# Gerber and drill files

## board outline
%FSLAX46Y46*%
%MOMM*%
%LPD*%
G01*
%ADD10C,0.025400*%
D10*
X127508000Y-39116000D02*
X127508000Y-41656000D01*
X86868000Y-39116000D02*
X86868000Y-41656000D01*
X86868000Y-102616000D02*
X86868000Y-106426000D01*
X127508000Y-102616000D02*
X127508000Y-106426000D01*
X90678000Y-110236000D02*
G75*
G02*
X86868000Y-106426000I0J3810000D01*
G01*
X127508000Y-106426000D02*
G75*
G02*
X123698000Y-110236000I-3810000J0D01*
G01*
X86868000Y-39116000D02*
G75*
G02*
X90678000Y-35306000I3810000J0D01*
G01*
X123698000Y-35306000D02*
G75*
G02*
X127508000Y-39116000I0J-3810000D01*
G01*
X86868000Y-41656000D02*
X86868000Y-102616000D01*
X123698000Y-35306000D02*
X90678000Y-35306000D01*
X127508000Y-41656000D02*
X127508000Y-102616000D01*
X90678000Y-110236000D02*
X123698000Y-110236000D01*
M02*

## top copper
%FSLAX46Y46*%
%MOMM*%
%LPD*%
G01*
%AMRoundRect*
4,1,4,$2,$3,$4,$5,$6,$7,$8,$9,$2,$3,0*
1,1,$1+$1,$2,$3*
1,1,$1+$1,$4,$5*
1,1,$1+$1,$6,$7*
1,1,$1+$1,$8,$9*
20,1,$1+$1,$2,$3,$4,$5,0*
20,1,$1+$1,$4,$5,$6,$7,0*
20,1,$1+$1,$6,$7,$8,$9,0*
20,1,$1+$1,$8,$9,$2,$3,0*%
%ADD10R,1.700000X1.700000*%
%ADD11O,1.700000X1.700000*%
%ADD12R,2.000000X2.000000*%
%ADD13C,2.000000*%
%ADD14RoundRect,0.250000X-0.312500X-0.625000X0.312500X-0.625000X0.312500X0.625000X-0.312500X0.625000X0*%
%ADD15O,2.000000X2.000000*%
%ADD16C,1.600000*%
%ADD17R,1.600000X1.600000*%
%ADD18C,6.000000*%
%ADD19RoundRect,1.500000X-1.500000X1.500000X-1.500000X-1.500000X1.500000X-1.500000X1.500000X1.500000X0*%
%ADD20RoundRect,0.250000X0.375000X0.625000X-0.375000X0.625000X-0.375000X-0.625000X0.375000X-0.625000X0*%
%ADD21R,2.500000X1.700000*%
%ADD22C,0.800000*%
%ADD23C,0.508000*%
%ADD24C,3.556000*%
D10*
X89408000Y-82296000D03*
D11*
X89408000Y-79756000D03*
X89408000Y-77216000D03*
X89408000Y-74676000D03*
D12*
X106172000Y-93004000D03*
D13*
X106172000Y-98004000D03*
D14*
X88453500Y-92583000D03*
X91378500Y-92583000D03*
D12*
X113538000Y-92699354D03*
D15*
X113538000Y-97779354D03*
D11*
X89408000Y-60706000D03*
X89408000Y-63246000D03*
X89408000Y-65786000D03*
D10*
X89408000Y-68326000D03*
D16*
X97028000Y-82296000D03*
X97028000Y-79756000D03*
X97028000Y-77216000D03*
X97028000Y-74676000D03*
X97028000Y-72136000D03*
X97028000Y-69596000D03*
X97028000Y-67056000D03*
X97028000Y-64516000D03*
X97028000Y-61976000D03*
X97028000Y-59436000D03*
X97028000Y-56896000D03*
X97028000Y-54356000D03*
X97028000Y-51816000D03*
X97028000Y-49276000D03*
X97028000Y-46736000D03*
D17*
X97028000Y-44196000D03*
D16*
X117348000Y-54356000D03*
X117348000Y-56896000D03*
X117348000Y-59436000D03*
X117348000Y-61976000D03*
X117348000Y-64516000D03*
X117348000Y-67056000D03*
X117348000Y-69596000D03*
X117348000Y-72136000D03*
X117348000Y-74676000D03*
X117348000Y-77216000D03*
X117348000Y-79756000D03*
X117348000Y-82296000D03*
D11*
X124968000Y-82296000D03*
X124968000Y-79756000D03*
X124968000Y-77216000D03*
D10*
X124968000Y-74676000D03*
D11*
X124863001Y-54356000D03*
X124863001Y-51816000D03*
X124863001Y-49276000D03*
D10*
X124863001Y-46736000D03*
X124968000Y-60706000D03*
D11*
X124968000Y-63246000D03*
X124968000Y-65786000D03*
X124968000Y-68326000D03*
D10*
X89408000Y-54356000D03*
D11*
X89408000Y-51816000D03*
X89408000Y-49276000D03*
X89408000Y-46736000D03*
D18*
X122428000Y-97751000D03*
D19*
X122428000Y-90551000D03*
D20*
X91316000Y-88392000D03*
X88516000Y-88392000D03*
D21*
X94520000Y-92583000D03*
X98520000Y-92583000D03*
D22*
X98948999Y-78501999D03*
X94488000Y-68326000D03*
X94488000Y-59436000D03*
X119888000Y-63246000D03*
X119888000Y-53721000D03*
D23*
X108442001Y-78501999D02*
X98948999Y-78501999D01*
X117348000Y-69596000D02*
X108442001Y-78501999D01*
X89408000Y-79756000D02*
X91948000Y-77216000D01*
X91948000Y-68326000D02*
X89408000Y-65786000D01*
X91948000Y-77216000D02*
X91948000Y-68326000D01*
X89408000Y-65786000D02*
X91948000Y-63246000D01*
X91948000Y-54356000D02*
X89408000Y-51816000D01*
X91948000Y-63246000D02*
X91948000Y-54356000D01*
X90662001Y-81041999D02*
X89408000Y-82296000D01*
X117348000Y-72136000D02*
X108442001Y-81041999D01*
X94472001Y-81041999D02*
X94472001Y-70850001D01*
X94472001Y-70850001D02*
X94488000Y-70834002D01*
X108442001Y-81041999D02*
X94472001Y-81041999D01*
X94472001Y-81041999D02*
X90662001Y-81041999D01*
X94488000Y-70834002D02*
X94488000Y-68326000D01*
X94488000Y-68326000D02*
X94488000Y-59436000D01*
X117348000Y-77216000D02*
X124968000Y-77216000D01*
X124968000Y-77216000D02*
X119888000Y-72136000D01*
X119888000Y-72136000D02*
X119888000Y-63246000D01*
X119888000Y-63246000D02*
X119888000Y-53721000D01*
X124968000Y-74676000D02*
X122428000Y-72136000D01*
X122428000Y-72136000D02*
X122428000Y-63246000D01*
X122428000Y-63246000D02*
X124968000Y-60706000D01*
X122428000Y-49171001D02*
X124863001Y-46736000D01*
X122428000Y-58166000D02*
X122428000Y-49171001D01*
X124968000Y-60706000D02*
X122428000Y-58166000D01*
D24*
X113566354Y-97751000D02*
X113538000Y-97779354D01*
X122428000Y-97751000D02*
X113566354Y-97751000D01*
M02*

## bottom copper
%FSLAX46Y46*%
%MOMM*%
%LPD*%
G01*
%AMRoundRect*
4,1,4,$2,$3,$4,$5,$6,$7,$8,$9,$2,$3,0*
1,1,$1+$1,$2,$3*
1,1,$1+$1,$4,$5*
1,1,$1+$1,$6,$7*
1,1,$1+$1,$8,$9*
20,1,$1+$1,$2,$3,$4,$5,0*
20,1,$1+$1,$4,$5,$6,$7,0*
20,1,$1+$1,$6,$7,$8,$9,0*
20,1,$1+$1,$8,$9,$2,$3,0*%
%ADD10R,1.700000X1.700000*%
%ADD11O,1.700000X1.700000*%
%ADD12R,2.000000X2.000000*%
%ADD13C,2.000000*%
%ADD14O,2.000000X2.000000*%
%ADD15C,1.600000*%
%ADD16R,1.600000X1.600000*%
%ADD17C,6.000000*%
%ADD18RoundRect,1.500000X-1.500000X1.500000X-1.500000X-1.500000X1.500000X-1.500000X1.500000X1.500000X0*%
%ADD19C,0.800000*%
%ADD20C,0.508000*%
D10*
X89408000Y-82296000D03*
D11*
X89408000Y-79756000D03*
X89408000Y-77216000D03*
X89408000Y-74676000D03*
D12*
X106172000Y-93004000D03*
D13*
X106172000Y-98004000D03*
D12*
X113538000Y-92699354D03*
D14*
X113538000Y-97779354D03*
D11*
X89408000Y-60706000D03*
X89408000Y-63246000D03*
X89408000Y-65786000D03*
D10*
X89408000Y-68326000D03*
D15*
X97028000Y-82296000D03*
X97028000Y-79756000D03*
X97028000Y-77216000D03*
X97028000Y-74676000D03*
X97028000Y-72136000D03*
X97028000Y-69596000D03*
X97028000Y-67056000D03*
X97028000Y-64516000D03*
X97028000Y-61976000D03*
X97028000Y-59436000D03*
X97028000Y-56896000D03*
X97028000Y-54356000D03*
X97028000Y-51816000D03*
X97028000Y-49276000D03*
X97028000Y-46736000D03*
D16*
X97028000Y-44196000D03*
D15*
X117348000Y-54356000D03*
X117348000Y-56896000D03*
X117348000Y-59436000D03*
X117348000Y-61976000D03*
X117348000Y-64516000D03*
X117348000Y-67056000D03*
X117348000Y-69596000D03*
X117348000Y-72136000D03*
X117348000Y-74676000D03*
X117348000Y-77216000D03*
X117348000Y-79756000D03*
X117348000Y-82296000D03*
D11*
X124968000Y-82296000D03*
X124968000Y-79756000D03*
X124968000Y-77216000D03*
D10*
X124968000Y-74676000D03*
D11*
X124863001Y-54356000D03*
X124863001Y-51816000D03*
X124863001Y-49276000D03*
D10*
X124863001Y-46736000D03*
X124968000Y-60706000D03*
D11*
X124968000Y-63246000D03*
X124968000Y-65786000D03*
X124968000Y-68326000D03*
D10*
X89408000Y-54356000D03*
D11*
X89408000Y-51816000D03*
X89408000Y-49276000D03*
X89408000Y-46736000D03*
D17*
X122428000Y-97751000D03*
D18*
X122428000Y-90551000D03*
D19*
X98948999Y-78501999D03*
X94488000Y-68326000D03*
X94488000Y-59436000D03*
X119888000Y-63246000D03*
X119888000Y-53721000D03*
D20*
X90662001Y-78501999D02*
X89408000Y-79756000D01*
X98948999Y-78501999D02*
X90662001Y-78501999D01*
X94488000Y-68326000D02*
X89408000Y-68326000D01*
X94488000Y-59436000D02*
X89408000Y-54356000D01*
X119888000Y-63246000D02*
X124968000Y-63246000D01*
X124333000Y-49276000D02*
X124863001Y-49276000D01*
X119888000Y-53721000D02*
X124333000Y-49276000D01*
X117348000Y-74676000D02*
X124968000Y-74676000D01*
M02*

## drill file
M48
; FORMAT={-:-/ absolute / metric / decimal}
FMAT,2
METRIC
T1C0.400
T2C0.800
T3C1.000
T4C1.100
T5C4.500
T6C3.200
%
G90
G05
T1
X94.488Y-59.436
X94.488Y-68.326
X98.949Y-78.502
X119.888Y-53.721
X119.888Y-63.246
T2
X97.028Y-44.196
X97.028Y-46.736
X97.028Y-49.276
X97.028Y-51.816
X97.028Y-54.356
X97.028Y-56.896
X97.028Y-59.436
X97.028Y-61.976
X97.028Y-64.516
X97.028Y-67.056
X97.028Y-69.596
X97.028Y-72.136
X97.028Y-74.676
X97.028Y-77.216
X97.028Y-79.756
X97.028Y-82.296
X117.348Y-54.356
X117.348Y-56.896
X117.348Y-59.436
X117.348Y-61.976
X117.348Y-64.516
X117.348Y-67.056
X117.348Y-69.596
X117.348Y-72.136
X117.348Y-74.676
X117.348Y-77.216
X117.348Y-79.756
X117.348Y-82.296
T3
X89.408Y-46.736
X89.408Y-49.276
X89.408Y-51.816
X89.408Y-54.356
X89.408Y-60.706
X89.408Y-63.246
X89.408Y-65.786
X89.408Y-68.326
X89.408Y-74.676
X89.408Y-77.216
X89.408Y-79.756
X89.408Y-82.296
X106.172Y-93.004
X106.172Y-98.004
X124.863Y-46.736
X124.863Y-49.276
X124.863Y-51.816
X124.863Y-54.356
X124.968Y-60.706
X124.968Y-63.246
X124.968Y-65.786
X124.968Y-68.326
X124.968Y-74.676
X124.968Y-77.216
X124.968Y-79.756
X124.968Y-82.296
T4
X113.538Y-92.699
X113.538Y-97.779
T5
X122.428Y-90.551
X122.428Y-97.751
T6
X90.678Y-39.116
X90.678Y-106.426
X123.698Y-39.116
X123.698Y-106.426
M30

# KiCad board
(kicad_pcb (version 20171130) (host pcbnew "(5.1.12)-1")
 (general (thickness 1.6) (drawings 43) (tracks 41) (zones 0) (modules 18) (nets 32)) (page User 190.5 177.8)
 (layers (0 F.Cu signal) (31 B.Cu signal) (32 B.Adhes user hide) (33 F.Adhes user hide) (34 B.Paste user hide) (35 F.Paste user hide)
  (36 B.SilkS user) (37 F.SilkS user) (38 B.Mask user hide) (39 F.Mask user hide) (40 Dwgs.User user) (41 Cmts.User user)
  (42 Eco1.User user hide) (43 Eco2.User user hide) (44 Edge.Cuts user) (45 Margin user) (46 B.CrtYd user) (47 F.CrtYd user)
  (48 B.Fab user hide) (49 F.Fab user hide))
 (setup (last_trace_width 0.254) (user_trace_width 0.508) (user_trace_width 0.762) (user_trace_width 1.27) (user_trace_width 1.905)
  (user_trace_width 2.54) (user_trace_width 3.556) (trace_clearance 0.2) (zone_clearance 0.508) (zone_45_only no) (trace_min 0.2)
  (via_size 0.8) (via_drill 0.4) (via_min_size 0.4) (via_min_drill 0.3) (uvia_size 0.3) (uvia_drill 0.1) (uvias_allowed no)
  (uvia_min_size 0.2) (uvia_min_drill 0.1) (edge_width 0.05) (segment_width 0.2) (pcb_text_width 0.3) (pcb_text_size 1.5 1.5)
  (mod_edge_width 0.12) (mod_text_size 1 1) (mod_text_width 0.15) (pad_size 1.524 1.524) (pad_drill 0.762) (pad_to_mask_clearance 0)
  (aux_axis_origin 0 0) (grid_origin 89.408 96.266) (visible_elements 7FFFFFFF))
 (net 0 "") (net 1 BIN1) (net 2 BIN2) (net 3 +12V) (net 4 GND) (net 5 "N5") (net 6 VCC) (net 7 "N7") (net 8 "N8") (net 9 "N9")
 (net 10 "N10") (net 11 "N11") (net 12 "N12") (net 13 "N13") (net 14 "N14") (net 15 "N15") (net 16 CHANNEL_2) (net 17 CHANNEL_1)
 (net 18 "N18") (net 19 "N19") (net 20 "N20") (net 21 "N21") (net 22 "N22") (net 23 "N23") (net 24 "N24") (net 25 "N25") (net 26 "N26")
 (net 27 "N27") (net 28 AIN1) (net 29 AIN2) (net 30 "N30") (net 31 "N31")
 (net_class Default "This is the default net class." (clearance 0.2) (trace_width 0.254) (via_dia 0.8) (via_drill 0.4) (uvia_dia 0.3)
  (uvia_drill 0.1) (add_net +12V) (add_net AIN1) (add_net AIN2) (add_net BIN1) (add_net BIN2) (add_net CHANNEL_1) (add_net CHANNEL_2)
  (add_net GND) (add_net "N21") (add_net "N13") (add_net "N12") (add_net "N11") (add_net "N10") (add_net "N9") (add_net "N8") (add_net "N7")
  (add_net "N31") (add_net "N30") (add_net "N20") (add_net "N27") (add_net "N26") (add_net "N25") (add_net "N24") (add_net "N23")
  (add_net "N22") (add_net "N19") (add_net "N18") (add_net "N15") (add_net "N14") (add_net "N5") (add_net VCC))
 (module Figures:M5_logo (layer F.Cu) (at 99.568 105.405088)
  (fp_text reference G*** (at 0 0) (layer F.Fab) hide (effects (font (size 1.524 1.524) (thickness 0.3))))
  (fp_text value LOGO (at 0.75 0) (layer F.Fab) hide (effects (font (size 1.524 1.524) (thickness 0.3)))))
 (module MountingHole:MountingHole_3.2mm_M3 (layer F.Cu) (at 123.698 39.116)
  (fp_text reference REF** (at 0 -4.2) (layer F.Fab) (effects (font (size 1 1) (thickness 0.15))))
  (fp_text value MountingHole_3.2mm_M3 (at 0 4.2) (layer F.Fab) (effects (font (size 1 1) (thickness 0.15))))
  (pad 1 np_thru_hole circle (at 0 0) (size 3.2 3.2) (drill 3.2) (layers *.Cu *.Mask)))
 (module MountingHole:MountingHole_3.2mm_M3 (layer F.Cu) (at 90.678 39.116)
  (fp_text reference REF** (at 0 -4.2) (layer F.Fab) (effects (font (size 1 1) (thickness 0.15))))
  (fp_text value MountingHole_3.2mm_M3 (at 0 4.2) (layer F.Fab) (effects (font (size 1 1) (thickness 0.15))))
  (pad 1 np_thru_hole circle (at 0 0) (size 3.2 3.2) (drill 3.2) (layers *.Cu *.Mask)))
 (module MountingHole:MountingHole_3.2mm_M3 (layer F.Cu) (at 123.698 106.426)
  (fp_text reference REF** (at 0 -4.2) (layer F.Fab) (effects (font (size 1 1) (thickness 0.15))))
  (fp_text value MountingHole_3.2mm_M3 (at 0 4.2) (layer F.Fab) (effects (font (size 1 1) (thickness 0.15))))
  (pad 1 np_thru_hole circle (at 0 0) (size 3.2 3.2) (drill 3.2) (layers *.Cu *.Mask)))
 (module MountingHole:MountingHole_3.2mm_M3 (layer F.Cu) (at 90.678 106.426)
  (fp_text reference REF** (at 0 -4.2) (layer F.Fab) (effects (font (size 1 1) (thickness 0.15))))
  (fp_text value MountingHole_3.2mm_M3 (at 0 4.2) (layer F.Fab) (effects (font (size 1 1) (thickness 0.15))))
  (pad 1 np_thru_hole circle (at 0 0) (size 3.2 3.2) (drill 3.2) (layers *.Cu *.Mask)))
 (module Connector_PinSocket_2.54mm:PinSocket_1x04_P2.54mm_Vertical (layer F.Cu) (at 89.408 82.296 180)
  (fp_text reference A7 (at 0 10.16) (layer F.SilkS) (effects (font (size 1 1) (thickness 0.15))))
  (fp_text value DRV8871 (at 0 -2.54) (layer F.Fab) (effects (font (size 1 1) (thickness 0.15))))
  (pad 1 thru_hole rect (at 0 0 180) (size 1.7 1.7) (drill 1) (layers *.Cu *.Mask) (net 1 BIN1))
  (pad 2 thru_hole oval (at 0 2.54 180) (size 1.7 1.7) (drill 1) (layers *.Cu *.Mask) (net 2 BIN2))
  (pad 3 thru_hole oval (at 0 5.08 180) (size 1.7 1.7) (drill 1) (layers *.Cu *.Mask) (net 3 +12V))
  (pad 4 thru_hole oval (at 0 7.62 180) (size 1.7 1.7) (drill 1) (layers *.Cu *.Mask) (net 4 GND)))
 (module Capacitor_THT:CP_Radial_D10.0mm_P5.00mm (layer F.Cu) (at 106.172 93.004 270)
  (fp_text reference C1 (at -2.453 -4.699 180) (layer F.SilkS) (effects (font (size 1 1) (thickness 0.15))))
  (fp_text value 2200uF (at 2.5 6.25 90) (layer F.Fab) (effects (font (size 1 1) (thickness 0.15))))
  (pad 1 thru_hole rect (at 0 0 270) (size 2 2) (drill 1) (layers *.Cu *.Mask) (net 3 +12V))
  (pad 2 thru_hole circle (at 5 0 270) (size 2 2) (drill 1) (layers *.Cu *.Mask) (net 4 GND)))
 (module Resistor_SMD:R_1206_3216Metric (layer F.Cu) (at 89.916 92.583)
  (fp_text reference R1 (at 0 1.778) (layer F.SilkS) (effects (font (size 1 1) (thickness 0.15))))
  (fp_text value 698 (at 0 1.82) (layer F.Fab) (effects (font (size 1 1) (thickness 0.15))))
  (pad 1 smd roundrect (at -1.4625 0) (size 1.125 1.75) (layers F.Cu F.Paste F.Mask) (roundrect_rratio 0.222222) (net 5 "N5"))
  (pad 2 smd roundrect (at 1.4625 0) (size 1.125 1.75) (layers F.Cu F.Paste F.Mask) (roundrect_rratio 0.222222) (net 3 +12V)))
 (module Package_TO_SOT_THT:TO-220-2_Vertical (layer F.Cu) (at 113.538 92.699354 270)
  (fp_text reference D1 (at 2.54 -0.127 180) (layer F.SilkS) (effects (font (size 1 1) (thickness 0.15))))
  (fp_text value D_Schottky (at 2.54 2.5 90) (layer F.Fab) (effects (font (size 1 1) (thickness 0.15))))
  (pad 1 thru_hole rect (at 0 0 270) (size 2 2) (drill 1.1) (layers *.Cu *.Mask) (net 3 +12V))
  (pad 2 thru_hole oval (at 5.08 0 270) (size 2 2) (drill 1.1) (layers *.Cu *.Mask) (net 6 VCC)))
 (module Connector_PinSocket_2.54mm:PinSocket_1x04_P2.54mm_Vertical (layer F.Cu) (at 89.408 68.326 180)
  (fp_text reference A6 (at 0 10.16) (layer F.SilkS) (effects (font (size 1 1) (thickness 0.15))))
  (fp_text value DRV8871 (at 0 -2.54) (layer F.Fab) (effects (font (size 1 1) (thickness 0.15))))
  (pad 4 thru_hole oval (at 0 7.62 180) (size 1.7 1.7) (drill 1) (layers *.Cu *.Mask) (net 4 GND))
  (pad 3 thru_hole oval (at 0 5.08 180) (size 1.7 1.7) (drill 1) (layers *.Cu *.Mask) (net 3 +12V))
  (pad 2 thru_hole oval (at 0 2.54 180) (size 1.7 1.7) (drill 1) (layers *.Cu *.Mask) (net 2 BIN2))
  (pad 1 thru_hole rect (at 0 0 180) (size 1.7 1.7) (drill 1) (layers *.Cu *.Mask) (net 1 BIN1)))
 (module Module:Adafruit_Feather (layer F.Cu) (at 97.028 44.196)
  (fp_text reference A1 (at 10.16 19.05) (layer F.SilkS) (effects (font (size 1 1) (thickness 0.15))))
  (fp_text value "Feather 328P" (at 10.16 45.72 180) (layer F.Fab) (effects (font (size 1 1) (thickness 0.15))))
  (pad 16 thru_hole circle (at 0 38.1 180) (size 1.6 1.6) (drill 0.8) (layers *.Cu *.Mask) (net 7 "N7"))
  (pad 15 thru_hole circle (at 0 35.56 180) (size 1.6 1.6) (drill 0.8) (layers *.Cu *.Mask) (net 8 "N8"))
  (pad 14 thru_hole circle (at 0 33.02 180) (size 1.6 1.6) (drill 0.8) (layers *.Cu *.Mask) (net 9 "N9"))
  (pad 13 thru_hole circle (at 0 30.48 180) (size 1.6 1.6) (drill 0.8) (layers *.Cu *.Mask) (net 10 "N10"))
  (pad 12 thru_hole circle (at 0 27.94 180) (size 1.6 1.6) (drill 0.8) (layers *.Cu *.Mask) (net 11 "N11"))
  (pad 11 thru_hole circle (at 0 25.4 180) (size 1.6 1.6) (drill 0.8) (layers *.Cu *.Mask) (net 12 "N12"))
  (pad 10 thru_hole circle (at 0 22.86 180) (size 1.6 1.6) (drill 0.8) (layers *.Cu *.Mask) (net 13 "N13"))
  (pad 9 thru_hole circle (at 0 20.32 180) (size 1.6 1.6) (drill 0.8) (layers *.Cu *.Mask) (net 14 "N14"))
  (pad 8 thru_hole circle (at 0 17.78 180) (size 1.6 1.6) (drill 0.8) (layers *.Cu *.Mask) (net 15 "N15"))
  (pad 7 thru_hole circle (at 0 15.24 180) (size 1.6 1.6) (drill 0.8) (layers *.Cu *.Mask) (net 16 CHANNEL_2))
  (pad 6 thru_hole circle (at 0 12.7 180) (size 1.6 1.6) (drill 0.8) (layers *.Cu *.Mask) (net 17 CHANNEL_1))
  (pad 5 thru_hole circle (at 0 10.16 180) (size 1.6 1.6) (drill 0.8) (layers *.Cu *.Mask) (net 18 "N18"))
  (pad 4 thru_hole circle (at 0 7.62 180) (size 1.6 1.6) (drill 0.8) (layers *.Cu *.Mask) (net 4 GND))
  (pad 3 thru_hole circle (at 0 5.08 180) (size 1.6 1.6) (drill 0.8) (layers *.Cu *.Mask) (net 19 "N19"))
  (pad 2 thru_hole circle (at 0 2.54 180) (size 1.6 1.6) (drill 0.8) (layers *.Cu *.Mask) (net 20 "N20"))
  (pad 1 thru_hole rect (at 0 0 180) (size 1.6 1.6) (drill 0.8) (layers *.Cu *.Mask) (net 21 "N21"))
  (pad 28 thru_hole circle (at 20.32 10.16 180) (size 1.6 1.6) (drill 0.8) (layers *.Cu *.Mask) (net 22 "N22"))
  (pad 27 thru_hole circle (at 20.32 12.7 180) (size 1.6 1.6) (drill 0.8) (layers *.Cu *.Mask) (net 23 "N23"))
  (pad 26 thru_hole circle (at 20.32 15.24 180) (size 1.6 1.6) (drill 0.8) (layers *.Cu *.Mask) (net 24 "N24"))
  (pad 25 thru_hole circle (at 20.32 17.78 180) (size 1.6 1.6) (drill 0.8) (layers *.Cu *.Mask) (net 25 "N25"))
  (pad 24 thru_hole circle (at 20.32 20.32 180) (size 1.6 1.6) (drill 0.8) (layers *.Cu *.Mask) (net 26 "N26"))
  (pad 23 thru_hole circle (at 20.32 22.86 180) (size 1.6 1.6) (drill 0.8) (layers *.Cu *.Mask) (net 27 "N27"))
  (pad 22 thru_hole circle (at 20.32 25.4 180) (size 1.6 1.6) (drill 0.8) (layers *.Cu *.Mask) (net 2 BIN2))
  (pad 21 thru_hole circle (at 20.32 27.94 180) (size 1.6 1.6) (drill 0.8) (layers *.Cu *.Mask) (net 1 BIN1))
  (pad 20 thru_hole circle (at 20.32 30.48 180) (size 1.6 1.6) (drill 0.8) (layers *.Cu *.Mask) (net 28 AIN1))
  (pad 19 thru_hole circle (at 20.32 33.02 180) (size 1.6 1.6) (drill 0.8) (layers *.Cu *.Mask) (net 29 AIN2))
  (pad 18 thru_hole circle (at 20.32 35.56 180) (size 1.6 1.6) (drill 0.8) (layers *.Cu *.Mask) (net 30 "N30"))
  (pad 17 thru_hole circle (at 20.32 38.1 180) (size 1.6 1.6) (drill 0.8) (layers *.Cu *.Mask) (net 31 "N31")))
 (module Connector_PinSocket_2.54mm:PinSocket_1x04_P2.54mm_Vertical (layer F.Cu) (at 124.968 74.676)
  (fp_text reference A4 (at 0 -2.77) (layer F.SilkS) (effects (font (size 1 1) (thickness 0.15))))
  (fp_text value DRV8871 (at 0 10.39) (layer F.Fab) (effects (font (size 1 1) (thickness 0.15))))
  (pad 4 thru_hole oval (at 0 7.62) (size 1.7 1.7) (drill 1) (layers *.Cu *.Mask) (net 4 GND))
  (pad 3 thru_hole oval (at 0 5.08) (size 1.7 1.7) (drill 1) (layers *.Cu *.Mask) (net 3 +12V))
  (pad 2 thru_hole oval (at 0 2.54) (size 1.7 1.7) (drill 1) (layers *.Cu *.Mask) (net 29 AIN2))
  (pad 1 thru_hole rect (at 0 0) (size 1.7 1.7) (drill 1) (layers *.Cu *.Mask) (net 28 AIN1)))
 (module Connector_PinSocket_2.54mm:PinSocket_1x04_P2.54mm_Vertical (layer F.Cu) (at 124.863001 46.736)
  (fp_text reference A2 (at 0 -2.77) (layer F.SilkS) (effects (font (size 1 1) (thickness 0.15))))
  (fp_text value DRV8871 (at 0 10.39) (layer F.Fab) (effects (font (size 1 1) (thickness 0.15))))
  (pad 4 thru_hole oval (at 0 7.62) (size 1.7 1.7) (drill 1) (layers *.Cu *.Mask) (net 4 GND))
  (pad 3 thru_hole oval (at 0 5.08) (size 1.7 1.7) (drill 1) (layers *.Cu *.Mask) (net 3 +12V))
  (pad 2 thru_hole oval (at 0 2.54) (size 1.7 1.7) (drill 1) (layers *.Cu *.Mask) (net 29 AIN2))
  (pad 1 thru_hole rect (at 0 0) (size 1.7 1.7) (drill 1) (layers *.Cu *.Mask) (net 28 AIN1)))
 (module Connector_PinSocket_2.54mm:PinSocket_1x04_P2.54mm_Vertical (layer F.Cu) (at 124.968 60.706)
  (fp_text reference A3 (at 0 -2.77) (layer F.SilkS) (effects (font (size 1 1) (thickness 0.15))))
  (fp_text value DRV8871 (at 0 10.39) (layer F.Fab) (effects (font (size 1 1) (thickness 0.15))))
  (pad 1 thru_hole rect (at 0 0) (size 1.7 1.7) (drill 1) (layers *.Cu *.Mask) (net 28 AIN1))
  (pad 2 thru_hole oval (at 0 2.54) (size 1.7 1.7) (drill 1) (layers *.Cu *.Mask) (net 29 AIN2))
  (pad 3 thru_hole oval (at 0 5.08) (size 1.7 1.7) (drill 1) (layers *.Cu *.Mask) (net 3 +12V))
  (pad 4 thru_hole oval (at 0 7.62) (size 1.7 1.7) (drill 1) (layers *.Cu *.Mask) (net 4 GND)))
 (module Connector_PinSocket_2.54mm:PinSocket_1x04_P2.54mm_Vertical (layer F.Cu) (at 89.408 54.356 180)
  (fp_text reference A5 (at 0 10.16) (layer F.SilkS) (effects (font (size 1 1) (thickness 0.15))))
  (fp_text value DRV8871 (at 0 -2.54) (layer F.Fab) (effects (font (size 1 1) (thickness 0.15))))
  (pad 1 thru_hole rect (at 0 0 180) (size 1.7 1.7) (drill 1) (layers *.Cu *.Mask) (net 1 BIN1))
  (pad 2 thru_hole oval (at 0 2.54 180) (size 1.7 1.7) (drill 1) (layers *.Cu *.Mask) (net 2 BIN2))
  (pad 3 thru_hole oval (at 0 5.08 180) (size 1.7 1.7) (drill 1) (layers *.Cu *.Mask) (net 3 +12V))
  (pad 4 thru_hole oval (at 0 7.62 180) (size 1.7 1.7) (drill 1) (layers *.Cu *.Mask) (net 4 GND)))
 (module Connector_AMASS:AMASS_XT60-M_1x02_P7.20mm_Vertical (layer F.Cu) (at 122.428 90.551 270)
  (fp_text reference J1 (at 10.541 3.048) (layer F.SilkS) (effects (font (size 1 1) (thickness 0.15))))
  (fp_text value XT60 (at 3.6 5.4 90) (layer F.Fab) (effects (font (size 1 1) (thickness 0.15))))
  (pad 2 thru_hole circle (at 7.2 0 270) (size 6 6) (drill 4.5) (layers *.Cu *.Mask) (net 6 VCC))
  (pad 1 thru_hole roundrect (at 0 0 270) (size 6 6) (drill 4.5) (layers *.Cu *.Mask) (roundrect_rratio 0.25) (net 4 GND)))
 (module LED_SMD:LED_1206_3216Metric (layer F.Cu) (at 89.916 88.392 180)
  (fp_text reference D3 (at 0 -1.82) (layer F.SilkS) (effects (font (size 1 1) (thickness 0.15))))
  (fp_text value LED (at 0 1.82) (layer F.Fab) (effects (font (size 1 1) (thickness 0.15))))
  (pad 1 smd roundrect (at -1.4 0 180) (size 1.25 1.75) (layers F.Cu F.Paste F.Mask) (roundrect_rratio 0.2) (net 4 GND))
  (pad 2 smd roundrect (at 1.4 0 180) (size 1.25 1.75) (layers F.Cu F.Paste F.Mask) (roundrect_rratio 0.2) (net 5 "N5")))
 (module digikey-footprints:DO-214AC (layer F.Cu) (at 96.52 92.583 180)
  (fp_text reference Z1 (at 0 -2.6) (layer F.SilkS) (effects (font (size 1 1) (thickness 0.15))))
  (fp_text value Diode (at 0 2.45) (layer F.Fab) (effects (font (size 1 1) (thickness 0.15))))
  (pad A smd rect (at 2 0 180) (size 2.5 1.7) (layers F.Cu F.Paste F.Mask) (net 4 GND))
  (pad K smd rect (at -2 0 180) (size 2.5 1.7) (layers F.Cu F.Paste F.Mask) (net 3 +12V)))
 (gr_line (start 127.508 39.116) (end 127.508 41.656) (layer Edge.Cuts) (width 0.0254))
 (gr_line (start 86.868 39.116) (end 86.868 41.656) (layer Edge.Cuts) (width 0.0254))
 (gr_line (start 86.868 102.616) (end 86.868 106.426) (layer Edge.Cuts) (width 0.0254))
 (gr_line (start 127.508 102.616) (end 127.508 106.426) (layer Edge.Cuts) (width 0.0254))
 (gr_arc (start 90.678 106.426) (end 86.868 106.426) (angle -90) (layer Edge.Cuts) (width 0.0254))
 (gr_arc (start 123.698 106.426) (end 123.698 110.236) (angle -90) (layer Edge.Cuts) (width 0.0254))
 (gr_arc (start 90.678 39.116) (end 90.678 35.306) (angle -90) (layer Edge.Cuts) (width 0.0254))
 (gr_arc (start 123.698 39.116) (end 127.508 39.116) (angle -90) (layer Edge.Cuts) (width 0.0254))
 (gr_line (start 86.868 41.656) (end 86.868 102.616) (layer Edge.Cuts) (width 0.0254))
 (gr_line (start 123.698 35.306) (end 90.678 35.306) (layer Edge.Cuts) (width 0.0254))
 (gr_line (start 127.508 41.656) (end 127.508 102.616) (layer Edge.Cuts) (width 0.0254))
 (gr_line (start 90.678 110.236) (end 123.698 110.236) (layer Edge.Cuts) (width 0.0254))
 (segment (start 108.442001 78.501999) (end 98.948999 78.501999) (width 0.508) (layer F.Cu) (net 2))
 (segment (start 117.348 69.596) (end 108.442001 78.501999) (width 0.508) (layer F.Cu) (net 2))
 (via (at 98.948999 78.501999) (size 0.8) (drill 0.4) (layers F.Cu B.Cu) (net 2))
 (segment (start 90.662001 78.501999) (end 89.408 79.756) (width 0.508) (layer B.Cu) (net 2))
 (segment (start 98.948999 78.501999) (end 90.662001 78.501999) (width 0.508) (layer B.Cu) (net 2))
 (segment (start 89.408 79.756) (end 91.948 77.216) (width 0.508) (layer F.Cu) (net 2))
 (segment (start 91.948 68.326) (end 89.408 65.786) (width 0.508) (layer F.Cu) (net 2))
 (segment (start 91.948 77.216) (end 91.948 68.326) (width 0.508) (layer F.Cu) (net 2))
 (segment (start 89.408 65.786) (end 91.948 63.246) (width 0.508) (layer F.Cu) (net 2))
 (segment (start 91.948 54.356) (end 89.408 51.816) (width 0.508) (layer F.Cu) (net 2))
 (segment (start 91.948 63.246) (end 91.948 54.356) (width 0.508) (layer F.Cu) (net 2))
 (segment (start 90.662001 81.041999) (end 89.408 82.296) (width 0.508) (layer F.Cu) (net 1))
 (segment (start 117.348 72.136) (end 108.442001 81.041999) (width 0.508) (layer F.Cu) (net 1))
 (segment (start 94.472001 81.041999) (end 94.472001 70.850001) (width 0.508) (layer F.Cu) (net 1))
 (segment (start 94.472001 70.850001) (end 94.488 70.834002) (width 0.508) (layer F.Cu) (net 1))
 (segment (start 108.442001 81.041999) (end 94.472001 81.041999) (width 0.508) (layer F.Cu) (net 1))
 (segment (start 94.472001 81.041999) (end 90.662001 81.041999) (width 0.508) (layer F.Cu) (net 1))
 (segment (start 94.488 70.834002) (end 94.488 68.326) (width 0.508) (layer F.Cu) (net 1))
 (via (at 94.488 68.326) (size 0.8) (drill 0.4) (layers F.Cu B.Cu) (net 1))
 (segment (start 94.488 68.326) (end 89.408 68.326) (width 0.508) (layer B.Cu) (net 1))
 (segment (start 94.488 68.326) (end 94.488 59.436) (width 0.508) (layer F.Cu) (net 1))
 (via (at 94.488 59.436) (size 0.8) (drill 0.4) (layers F.Cu B.Cu) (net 1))
 (segment (start 94.488 59.436) (end 89.408 54.356) (width 0.508) (layer B.Cu) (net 1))
 (segment (start 117.348 77.216) (end 124.968 77.216) (width 0.508) (layer F.Cu) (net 29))
 (segment (start 124.968 77.216) (end 119.888 72.136) (width 0.508) (layer F.Cu) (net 29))
 (segment (start 119.888 72.136) (end 119.888 63.246) (width 0.508) (layer F.Cu) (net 29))
 (via (at 119.888 63.246) (size 0.8) (drill 0.4) (layers F.Cu B.Cu) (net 29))
 (segment (start 119.888 63.246) (end 124.968 63.246) (width 0.508) (layer B.Cu) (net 29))
 (segment (start 119.888 63.246) (end 119.888 53.721) (width 0.508) (layer F.Cu) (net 29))
 (via (at 119.888 53.721) (size 0.8) (drill 0.4) (layers F.Cu B.Cu) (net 29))
 (segment (start 124.333 49.276) (end 124.863001 49.276) (width 0.508) (layer B.Cu) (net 29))
 (segment (start 119.888 53.721) (end 124.333 49.276) (width 0.508) (layer B.Cu) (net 29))
 (segment (start 117.348 74.676) (end 124.968 74.676) (width 0.508) (layer B.Cu) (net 28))
 (segment (start 124.968 74.676) (end 122.428 72.136) (width 0.508) (layer F.Cu) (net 28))
 (segment (start 122.428 72.136) (end 122.428 63.246) (width 0.508) (layer F.Cu) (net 28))
 (segment (start 122.428 63.246) (end 124.968 60.706) (width 0.508) (layer F.Cu) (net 28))
 (segment (start 122.428 49.171001) (end 124.863001 46.736) (width 0.508) (layer F.Cu) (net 28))
 (segment (start 122.428 58.166) (end 122.428 49.171001) (width 0.508) (layer F.Cu) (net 28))
 (segment (start 124.968 60.706) (end 122.428 58.166) (width 0.508) (layer F.Cu) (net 28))
 (segment (start 113.566354 97.751) (end 113.538 97.779354) (width 3.556) (layer F.Cu) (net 6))
 (segment (start 122.428 97.751) (end 113.566354 97.751) (width 3.556) (layer F.Cu) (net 6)))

